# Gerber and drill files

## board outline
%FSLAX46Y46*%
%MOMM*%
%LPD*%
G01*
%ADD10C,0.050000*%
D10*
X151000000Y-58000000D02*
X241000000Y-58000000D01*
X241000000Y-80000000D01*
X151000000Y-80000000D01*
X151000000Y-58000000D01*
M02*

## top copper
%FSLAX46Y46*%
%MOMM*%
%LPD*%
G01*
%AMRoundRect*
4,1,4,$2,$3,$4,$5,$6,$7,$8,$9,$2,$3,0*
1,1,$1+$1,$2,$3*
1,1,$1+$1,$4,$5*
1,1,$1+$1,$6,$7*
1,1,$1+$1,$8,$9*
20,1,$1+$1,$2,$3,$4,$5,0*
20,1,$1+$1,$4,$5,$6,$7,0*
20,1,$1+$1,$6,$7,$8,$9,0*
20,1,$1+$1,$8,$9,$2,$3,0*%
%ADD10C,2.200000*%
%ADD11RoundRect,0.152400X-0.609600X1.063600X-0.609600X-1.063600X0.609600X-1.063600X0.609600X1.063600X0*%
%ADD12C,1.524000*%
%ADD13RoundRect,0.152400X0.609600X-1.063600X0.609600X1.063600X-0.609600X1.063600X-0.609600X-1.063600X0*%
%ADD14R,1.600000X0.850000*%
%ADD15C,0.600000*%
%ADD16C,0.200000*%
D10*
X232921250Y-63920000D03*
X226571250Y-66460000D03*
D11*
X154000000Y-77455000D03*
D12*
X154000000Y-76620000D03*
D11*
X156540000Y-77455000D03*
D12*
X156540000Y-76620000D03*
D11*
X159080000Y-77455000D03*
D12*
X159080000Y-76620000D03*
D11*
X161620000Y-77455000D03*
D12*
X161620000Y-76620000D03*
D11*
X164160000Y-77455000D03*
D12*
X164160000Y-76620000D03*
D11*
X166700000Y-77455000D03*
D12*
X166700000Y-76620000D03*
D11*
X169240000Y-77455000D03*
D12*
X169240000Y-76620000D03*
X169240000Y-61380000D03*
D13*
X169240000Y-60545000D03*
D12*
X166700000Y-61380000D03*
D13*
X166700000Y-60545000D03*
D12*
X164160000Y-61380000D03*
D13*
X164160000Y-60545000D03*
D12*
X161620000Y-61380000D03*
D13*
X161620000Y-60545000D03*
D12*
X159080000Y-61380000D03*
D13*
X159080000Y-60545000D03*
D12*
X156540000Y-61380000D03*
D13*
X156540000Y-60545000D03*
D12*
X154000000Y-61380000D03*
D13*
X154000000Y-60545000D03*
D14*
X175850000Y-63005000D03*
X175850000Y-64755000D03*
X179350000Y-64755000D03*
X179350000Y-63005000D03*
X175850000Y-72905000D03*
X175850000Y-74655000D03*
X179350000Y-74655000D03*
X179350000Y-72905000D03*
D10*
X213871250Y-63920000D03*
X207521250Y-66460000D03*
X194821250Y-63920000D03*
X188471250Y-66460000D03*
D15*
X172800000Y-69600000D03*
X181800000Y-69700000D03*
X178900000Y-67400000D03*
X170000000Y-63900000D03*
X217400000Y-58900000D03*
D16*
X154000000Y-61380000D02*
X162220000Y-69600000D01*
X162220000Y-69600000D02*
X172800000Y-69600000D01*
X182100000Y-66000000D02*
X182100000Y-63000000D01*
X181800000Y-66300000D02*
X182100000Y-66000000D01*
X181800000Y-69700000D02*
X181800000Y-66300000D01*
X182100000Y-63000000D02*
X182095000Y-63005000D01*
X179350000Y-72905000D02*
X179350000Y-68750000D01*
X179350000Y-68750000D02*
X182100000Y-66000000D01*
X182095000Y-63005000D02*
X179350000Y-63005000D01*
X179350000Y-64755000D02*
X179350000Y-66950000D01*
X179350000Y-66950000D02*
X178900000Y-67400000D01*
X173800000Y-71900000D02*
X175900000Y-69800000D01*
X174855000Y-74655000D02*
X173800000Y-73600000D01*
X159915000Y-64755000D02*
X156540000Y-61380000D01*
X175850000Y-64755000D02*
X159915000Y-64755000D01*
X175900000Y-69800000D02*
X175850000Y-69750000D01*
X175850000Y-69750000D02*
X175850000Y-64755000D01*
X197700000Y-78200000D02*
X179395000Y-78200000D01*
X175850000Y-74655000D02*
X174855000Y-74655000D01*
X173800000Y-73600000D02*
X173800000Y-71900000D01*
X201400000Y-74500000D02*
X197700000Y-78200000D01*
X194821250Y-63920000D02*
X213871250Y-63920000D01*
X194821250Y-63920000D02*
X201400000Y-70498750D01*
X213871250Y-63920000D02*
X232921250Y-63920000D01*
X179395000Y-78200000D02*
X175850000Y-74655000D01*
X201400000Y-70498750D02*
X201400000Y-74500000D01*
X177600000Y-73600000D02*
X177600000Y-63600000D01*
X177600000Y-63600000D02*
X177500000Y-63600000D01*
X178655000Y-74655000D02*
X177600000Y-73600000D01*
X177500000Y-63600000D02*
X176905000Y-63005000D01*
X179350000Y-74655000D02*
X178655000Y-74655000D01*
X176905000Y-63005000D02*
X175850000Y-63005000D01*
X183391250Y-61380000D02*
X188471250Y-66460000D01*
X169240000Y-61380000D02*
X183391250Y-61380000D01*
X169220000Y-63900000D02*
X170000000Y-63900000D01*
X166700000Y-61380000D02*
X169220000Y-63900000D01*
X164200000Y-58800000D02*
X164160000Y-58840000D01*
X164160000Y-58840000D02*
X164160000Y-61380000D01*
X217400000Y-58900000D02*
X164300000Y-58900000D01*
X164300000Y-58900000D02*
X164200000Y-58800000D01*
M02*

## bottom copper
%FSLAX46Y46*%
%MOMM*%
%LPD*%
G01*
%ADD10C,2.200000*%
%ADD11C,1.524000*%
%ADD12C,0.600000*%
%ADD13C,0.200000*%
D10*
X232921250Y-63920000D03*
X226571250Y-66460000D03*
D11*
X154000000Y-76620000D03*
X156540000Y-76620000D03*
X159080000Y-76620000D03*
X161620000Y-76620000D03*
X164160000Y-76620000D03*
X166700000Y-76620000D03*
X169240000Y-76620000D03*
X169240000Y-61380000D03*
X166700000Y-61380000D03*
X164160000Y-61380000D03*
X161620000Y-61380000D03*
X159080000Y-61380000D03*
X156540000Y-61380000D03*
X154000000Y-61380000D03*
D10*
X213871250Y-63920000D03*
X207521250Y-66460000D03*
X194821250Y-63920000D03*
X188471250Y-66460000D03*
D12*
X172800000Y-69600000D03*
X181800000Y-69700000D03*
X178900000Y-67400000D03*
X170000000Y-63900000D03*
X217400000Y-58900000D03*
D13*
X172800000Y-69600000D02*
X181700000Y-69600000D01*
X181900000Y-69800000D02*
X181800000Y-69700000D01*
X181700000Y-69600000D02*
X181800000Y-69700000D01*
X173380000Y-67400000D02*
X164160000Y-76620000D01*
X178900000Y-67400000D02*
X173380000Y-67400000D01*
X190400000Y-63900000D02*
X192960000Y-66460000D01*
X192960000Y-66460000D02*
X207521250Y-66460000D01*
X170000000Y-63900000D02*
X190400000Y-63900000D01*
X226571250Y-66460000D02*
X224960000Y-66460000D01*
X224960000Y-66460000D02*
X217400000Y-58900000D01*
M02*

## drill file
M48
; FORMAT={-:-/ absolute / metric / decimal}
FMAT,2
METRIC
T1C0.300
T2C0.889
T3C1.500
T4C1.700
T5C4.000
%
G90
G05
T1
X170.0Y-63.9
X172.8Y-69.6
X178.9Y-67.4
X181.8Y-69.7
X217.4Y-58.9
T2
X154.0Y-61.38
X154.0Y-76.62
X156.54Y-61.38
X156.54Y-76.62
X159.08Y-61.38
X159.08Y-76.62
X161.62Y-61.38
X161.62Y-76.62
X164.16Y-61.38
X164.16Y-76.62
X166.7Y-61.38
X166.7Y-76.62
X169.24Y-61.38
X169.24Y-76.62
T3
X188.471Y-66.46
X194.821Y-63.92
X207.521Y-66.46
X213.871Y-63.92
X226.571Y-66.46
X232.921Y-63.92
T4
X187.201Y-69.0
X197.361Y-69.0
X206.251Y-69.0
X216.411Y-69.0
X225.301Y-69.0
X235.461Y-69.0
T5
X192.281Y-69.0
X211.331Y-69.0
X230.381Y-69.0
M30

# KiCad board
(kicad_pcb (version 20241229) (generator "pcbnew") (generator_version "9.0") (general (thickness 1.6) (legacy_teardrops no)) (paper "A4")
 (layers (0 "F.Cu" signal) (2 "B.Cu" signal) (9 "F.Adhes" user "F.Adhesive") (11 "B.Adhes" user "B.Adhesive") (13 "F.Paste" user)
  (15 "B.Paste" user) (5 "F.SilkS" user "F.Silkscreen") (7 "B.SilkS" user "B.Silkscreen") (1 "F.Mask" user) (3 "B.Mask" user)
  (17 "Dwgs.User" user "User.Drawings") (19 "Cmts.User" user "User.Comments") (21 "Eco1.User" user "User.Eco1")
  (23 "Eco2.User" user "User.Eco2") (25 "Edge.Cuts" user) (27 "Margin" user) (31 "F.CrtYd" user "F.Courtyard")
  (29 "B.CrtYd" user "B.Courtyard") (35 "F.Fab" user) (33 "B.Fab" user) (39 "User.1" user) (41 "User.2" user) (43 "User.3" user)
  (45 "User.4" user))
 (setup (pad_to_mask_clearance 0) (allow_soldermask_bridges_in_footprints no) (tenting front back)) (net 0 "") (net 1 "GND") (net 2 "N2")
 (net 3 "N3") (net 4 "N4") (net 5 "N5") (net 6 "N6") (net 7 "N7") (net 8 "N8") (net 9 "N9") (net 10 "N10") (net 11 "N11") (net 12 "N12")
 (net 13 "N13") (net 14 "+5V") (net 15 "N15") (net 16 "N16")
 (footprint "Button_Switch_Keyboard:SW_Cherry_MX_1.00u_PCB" (layer "F.Cu") (at 232.92125 63.92)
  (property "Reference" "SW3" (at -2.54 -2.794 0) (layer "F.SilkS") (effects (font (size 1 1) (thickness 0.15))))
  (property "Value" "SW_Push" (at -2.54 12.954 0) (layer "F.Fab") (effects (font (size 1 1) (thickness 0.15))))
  (pad "" np_thru_hole circle (at -7.62 5.08) (size 1.7 1.7) (drill 1.7) (layers "*.Cu" "*.Mask"))
  (pad "" np_thru_hole circle (at -2.54 5.08) (size 4 4) (drill 4) (layers "*.Cu" "*.Mask"))
  (pad "" np_thru_hole circle (at 2.54 5.08) (size 1.7 1.7) (drill 1.7) (layers "*.Cu" "*.Mask"))
  (pad "1" thru_hole circle (at 0 0) (size 2.2 2.2) (drill 1.5) (layers "*.Cu" "*.Mask") (remove_unused_layers no) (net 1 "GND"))
  (pad "2" thru_hole circle (at -6.35 2.54) (size 2.2 2.2) (drill 1.5) (layers "*.Cu" "*.Mask") (remove_unused_layers no) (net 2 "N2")))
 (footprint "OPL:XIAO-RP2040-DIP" (layer "F.Cu") (at 161.62 69 90)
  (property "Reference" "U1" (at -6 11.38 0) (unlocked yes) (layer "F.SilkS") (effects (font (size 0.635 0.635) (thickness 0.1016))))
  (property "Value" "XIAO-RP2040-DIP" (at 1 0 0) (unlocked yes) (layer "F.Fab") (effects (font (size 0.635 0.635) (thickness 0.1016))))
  (pad "1" smd roundrect (at -8.455 -7.62 270) (size 2.432 1.524) (layers "F.Cu" "F.Mask") (roundrect_rratio 0.1) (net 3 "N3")
   (thermal_bridge_angle 45))
  (pad "1" thru_hole circle (at -7.62 -7.62 270) (size 1.524 1.524) (drill 0.889) (layers "*.Cu" "*.Mask") (remove_unused_layers no)
   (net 3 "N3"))
  (pad "2" smd roundrect (at -8.455 -5.08 270) (size 2.432 1.524) (layers "F.Cu" "F.Mask") (roundrect_rratio 0.1) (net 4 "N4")
   (thermal_bridge_angle 45))
  (pad "2" thru_hole circle (at -7.62 -5.08 270) (size 1.524 1.524) (drill 0.889) (layers "*.Cu" "*.Mask") (remove_unused_layers no)
   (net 4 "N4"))
  (pad "3" smd roundrect (at -8.455 -2.54 270) (size 2.432 1.524) (layers "F.Cu" "F.Mask") (roundrect_rratio 0.1) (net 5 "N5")
   (thermal_bridge_angle 45))
  (pad "3" thru_hole circle (at -7.62 -2.54 270) (size 1.524 1.524) (drill 0.889) (layers "*.Cu" "*.Mask") (remove_unused_layers no)
   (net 5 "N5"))
  (pad "4" smd roundrect (at -8.455 0 270) (size 2.432 1.524) (layers "F.Cu" "F.Mask") (roundrect_rratio 0.1) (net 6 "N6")
   (thermal_bridge_angle 45))
  (pad "4" thru_hole circle (at -7.62 0 270) (size 1.524 1.524) (drill 0.889) (layers "*.Cu" "*.Mask") (remove_unused_layers no)
   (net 6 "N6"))
  (pad "5" smd roundrect (at -8.455 2.54 270) (size 2.432 1.524) (layers "F.Cu" "F.Mask") (roundrect_rratio 0.1) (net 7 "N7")
   (thermal_bridge_angle 45))
  (pad "5" thru_hole circle (at -7.62 2.54 270) (size 1.524 1.524) (drill 0.889) (layers "*.Cu" "*.Mask") (remove_unused_layers no)
   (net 7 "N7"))
  (pad "6" smd roundrect (at -8.455 5.08 270) (size 2.432 1.524) (layers "F.Cu" "F.Mask") (roundrect_rratio 0.1) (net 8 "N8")
   (thermal_bridge_angle 45))
  (pad "6" thru_hole circle (at -7.62 5.08 270) (size 1.524 1.524) (drill 0.889) (layers "*.Cu" "*.Mask") (remove_unused_layers no)
   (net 8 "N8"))
  (pad "7" smd roundrect (at -8.455 7.62 270) (size 2.432 1.524) (layers "F.Cu" "F.Mask") (roundrect_rratio 0.1) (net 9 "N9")
   (thermal_bridge_angle 45))
  (pad "7" thru_hole circle (at -7.62 7.62 270) (size 1.524 1.524) (drill 0.889) (layers "*.Cu" "*.Mask") (remove_unused_layers no)
   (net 9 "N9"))
  (pad "8" thru_hole circle (at 7.62 7.62 90) (size 1.524 1.524) (drill 0.889) (layers "*.Cu" "*.Mask") (remove_unused_layers no)
   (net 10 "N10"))
  (pad "8" smd roundrect (at 8.455 7.62 90) (size 2.432 1.524) (layers "F.Cu" "F.Mask") (roundrect_rratio 0.1) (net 10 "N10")
   (thermal_bridge_angle 45))
  (pad "9" thru_hole circle (at 7.62 5.08 90) (size 1.524 1.524) (drill 0.889) (layers "*.Cu" "*.Mask") (remove_unused_layers no)
   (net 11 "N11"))
  (pad "9" smd roundrect (at 8.455 5.08 90) (size 2.432 1.524) (layers "F.Cu" "F.Mask") (roundrect_rratio 0.1) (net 11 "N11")
   (thermal_bridge_angle 45))
  (pad "10" thru_hole circle (at 7.62 2.54 90) (size 1.524 1.524) (drill 0.889) (layers "*.Cu" "*.Mask") (remove_unused_layers no)
   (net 2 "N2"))
  (pad "10" smd roundrect (at 8.455 2.54 90) (size 2.432 1.524) (layers "F.Cu" "F.Mask") (roundrect_rratio 0.1) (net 2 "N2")
   (thermal_bridge_angle 45))
  (pad "11" thru_hole circle (at 7.62 0 90) (size 1.524 1.524) (drill 0.889) (layers "*.Cu" "*.Mask") (remove_unused_layers no)
   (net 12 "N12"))
  (pad "11" smd roundrect (at 8.455 0 90) (size 2.432 1.524) (layers "F.Cu" "F.Mask") (roundrect_rratio 0.1) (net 12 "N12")
   (thermal_bridge_angle 45))
  (pad "12" thru_hole circle (at 7.62 -2.54 90) (size 1.524 1.524) (drill 0.889) (layers "*.Cu" "*.Mask") (remove_unused_layers no)
   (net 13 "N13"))
  (pad "12" smd roundrect (at 8.455 -2.54 90) (size 2.432 1.524) (layers "F.Cu" "F.Mask") (roundrect_rratio 0.1) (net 13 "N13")
   (thermal_bridge_angle 45))
  (pad "13" thru_hole circle (at 7.62 -5.08 90) (size 1.524 1.524) (drill 0.889) (layers "*.Cu" "*.Mask") (remove_unused_layers no)
   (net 1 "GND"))
  (pad "13" smd roundrect (at 8.455 -5.08 90) (size 2.432 1.524) (layers "F.Cu" "F.Mask") (roundrect_rratio 0.1) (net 1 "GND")
   (thermal_bridge_angle 45))
  (pad "14" thru_hole circle (at 7.62 -7.62 90) (size 1.524 1.524) (drill 0.889) (layers "*.Cu" "*.Mask") (remove_unused_layers no)
   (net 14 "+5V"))
  (pad "14" smd roundrect (at 8.455 -7.62 90) (size 2.432 1.524) (layers "F.Cu" "F.Mask") (roundrect_rratio 0.1) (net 14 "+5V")
   (thermal_bridge_angle 45)))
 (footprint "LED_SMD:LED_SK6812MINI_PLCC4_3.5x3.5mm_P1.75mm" (layer "F.Cu") (at 177.6 63.88)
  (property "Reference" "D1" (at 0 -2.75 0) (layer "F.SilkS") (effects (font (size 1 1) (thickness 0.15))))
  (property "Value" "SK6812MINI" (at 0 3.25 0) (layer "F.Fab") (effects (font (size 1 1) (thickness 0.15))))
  (pad "1" smd rect (at -1.75 -0.875) (size 1.6 0.85) (layers "F.Cu" "F.Mask" "F.Paste") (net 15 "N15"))
  (pad "2" smd rect (at -1.75 0.875) (size 1.6 0.85) (layers "F.Cu" "F.Mask" "F.Paste") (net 1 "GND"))
  (pad "3" smd rect (at 1.75 0.875) (size 1.6 0.85) (layers "F.Cu" "F.Mask" "F.Paste") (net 7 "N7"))
  (pad "4" smd rect (at 1.75 -0.875) (size 1.6 0.85) (layers "F.Cu" "F.Mask" "F.Paste") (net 14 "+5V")))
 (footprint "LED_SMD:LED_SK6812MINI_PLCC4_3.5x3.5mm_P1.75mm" (layer "F.Cu") (at 177.6 73.78)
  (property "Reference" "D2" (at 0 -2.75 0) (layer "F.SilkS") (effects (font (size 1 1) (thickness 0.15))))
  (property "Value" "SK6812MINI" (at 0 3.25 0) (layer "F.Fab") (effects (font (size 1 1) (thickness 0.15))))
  (pad "1" smd rect (at -1.75 -0.875) (size 1.6 0.85) (layers "F.Cu" "F.Mask" "F.Paste") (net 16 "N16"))
  (pad "2" smd rect (at -1.75 0.875) (size 1.6 0.85) (layers "F.Cu" "F.Mask" "F.Paste") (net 1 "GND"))
  (pad "3" smd rect (at 1.75 0.875) (size 1.6 0.85) (layers "F.Cu" "F.Mask" "F.Paste") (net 15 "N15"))
  (pad "4" smd rect (at 1.75 -0.875) (size 1.6 0.85) (layers "F.Cu" "F.Mask" "F.Paste") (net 14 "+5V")))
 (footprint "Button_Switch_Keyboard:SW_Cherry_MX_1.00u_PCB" (layer "F.Cu") (at 213.87125 63.92)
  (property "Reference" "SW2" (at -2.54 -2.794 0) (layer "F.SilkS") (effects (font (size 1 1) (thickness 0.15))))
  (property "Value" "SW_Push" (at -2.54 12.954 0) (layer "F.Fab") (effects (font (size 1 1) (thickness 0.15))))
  (pad "" np_thru_hole circle (at -7.62 5.08) (size 1.7 1.7) (drill 1.7) (layers "*.Cu" "*.Mask"))
  (pad "" np_thru_hole circle (at -2.54 5.08) (size 4 4) (drill 4) (layers "*.Cu" "*.Mask"))
  (pad "" np_thru_hole circle (at 2.54 5.08) (size 1.7 1.7) (drill 1.7) (layers "*.Cu" "*.Mask"))
  (pad "1" thru_hole circle (at 0 0) (size 2.2 2.2) (drill 1.5) (layers "*.Cu" "*.Mask") (remove_unused_layers no) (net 1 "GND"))
  (pad "2" thru_hole circle (at -6.35 2.54) (size 2.2 2.2) (drill 1.5) (layers "*.Cu" "*.Mask") (remove_unused_layers no) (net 11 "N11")))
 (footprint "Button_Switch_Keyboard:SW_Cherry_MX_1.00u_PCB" (layer "F.Cu") (at 194.82125 63.92)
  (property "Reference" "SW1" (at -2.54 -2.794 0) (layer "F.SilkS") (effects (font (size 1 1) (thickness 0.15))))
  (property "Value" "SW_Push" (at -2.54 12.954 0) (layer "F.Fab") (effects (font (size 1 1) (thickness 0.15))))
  (pad "" np_thru_hole circle (at -7.62 5.08) (size 1.7 1.7) (drill 1.7) (layers "*.Cu" "*.Mask"))
  (pad "" np_thru_hole circle (at -2.54 5.08) (size 4 4) (drill 4) (layers "*.Cu" "*.Mask"))
  (pad "" np_thru_hole circle (at 2.54 5.08) (size 1.7 1.7) (drill 1.7) (layers "*.Cu" "*.Mask"))
  (pad "1" thru_hole circle (at 0 0) (size 2.2 2.2) (drill 1.5) (layers "*.Cu" "*.Mask") (remove_unused_layers no) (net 1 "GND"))
  (pad "2" thru_hole circle (at -6.35 2.54) (size 2.2 2.2) (drill 1.5) (layers "*.Cu" "*.Mask") (remove_unused_layers no) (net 10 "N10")))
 (gr_rect (start 151 58) (end 241 80) (stroke (width 0.05) (type default)) (fill no) (layer "Edge.Cuts"))
 (segment (start 154 61.38) (end 162.22 69.6) (width 0.2) (layer "F.Cu") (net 14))
 (segment (start 162.22 69.6) (end 172.8 69.6) (width 0.2) (layer "F.Cu") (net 14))
 (segment (start 182.1 66) (end 182.1 63) (width 0.2) (layer "F.Cu") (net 14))
 (segment (start 181.8 66.3) (end 182.1 66) (width 0.2) (layer "F.Cu") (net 14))
 (segment (start 181.8 69.7) (end 181.8 66.3) (width 0.2) (layer "F.Cu") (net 14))
 (segment (start 182.1 63) (end 182.095 63.005) (width 0.2) (layer "F.Cu") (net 14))
 (segment (start 179.35 72.905) (end 179.35 68.75) (width 0.2) (layer "F.Cu") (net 14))
 (segment (start 179.35 68.75) (end 182.1 66) (width 0.2) (layer "F.Cu") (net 14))
 (segment (start 182.095 63.005) (end 179.35 63.005) (width 0.2) (layer "F.Cu") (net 14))
 (via (at 172.8 69.6) (size 0.6) (drill 0.3) (layers "F.Cu" "B.Cu") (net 14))
 (via (at 181.8 69.7) (size 0.6) (drill 0.3) (layers "F.Cu" "B.Cu") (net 14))
 (segment (start 172.8 69.6) (end 181.7 69.6) (width 0.2) (layer "B.Cu") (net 14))
 (segment (start 181.9 69.8) (end 181.8 69.7) (width 0.2) (layer "B.Cu") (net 14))
 (segment (start 181.7 69.6) (end 181.8 69.7) (width 0.2) (layer "B.Cu") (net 14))
 (segment (start 179.35 64.755) (end 179.35 66.95) (width 0.2) (layer "F.Cu") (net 7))
 (segment (start 179.35 66.95) (end 178.9 67.4) (width 0.2) (layer "F.Cu") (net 7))
 (via (at 178.9 67.4) (size 0.6) (drill 0.3) (layers "F.Cu" "B.Cu") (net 7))
 (segment (start 173.38 67.4) (end 164.16 76.62) (width 0.2) (layer "B.Cu") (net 7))
 (segment (start 178.9 67.4) (end 173.38 67.4) (width 0.2) (layer "B.Cu") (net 7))
 (segment (start 173.8 71.9) (end 175.9 69.8) (width 0.2) (layer "F.Cu") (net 1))
 (segment (start 174.855 74.655) (end 173.8 73.6) (width 0.2) (layer "F.Cu") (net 1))
 (segment (start 159.915 64.755) (end 156.54 61.38) (width 0.2) (layer "F.Cu") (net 1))
 (segment (start 175.85 64.755) (end 159.915 64.755) (width 0.2) (layer "F.Cu") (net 1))
 (segment (start 175.9 69.8) (end 175.85 69.75) (width 0.2) (layer "F.Cu") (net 1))
 (segment (start 175.85 69.75) (end 175.85 64.755) (width 0.2) (layer "F.Cu") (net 1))
 (segment (start 197.7 78.2) (end 179.395 78.2) (width 0.2) (layer "F.Cu") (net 1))
 (segment (start 175.85 74.655) (end 174.855 74.655) (width 0.2) (layer "F.Cu") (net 1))
 (segment (start 173.8 73.6) (end 173.8 71.9) (width 0.2) (layer "F.Cu") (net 1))
 (segment (start 201.4 74.5) (end 197.7 78.2) (width 0.2) (layer "F.Cu") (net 1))
 (segment (start 194.82125 63.92) (end 213.87125 63.92) (width 0.2) (layer "F.Cu") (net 1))
 (segment (start 194.82125 63.92) (end 201.4 70.49875) (width 0.2) (layer "F.Cu") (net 1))
 (segment (start 213.87125 63.92) (end 232.92125 63.92) (width 0.2) (layer "F.Cu") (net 1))
 (segment (start 179.395 78.2) (end 175.85 74.655) (width 0.2) (layer "F.Cu") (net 1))
 (segment (start 201.4 70.49875) (end 201.4 74.5) (width 0.2) (layer "F.Cu") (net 1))
 (segment (start 177.6 73.6) (end 177.6 63.6) (width 0.2) (layer "F.Cu") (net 15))
 (segment (start 177.6 63.6) (end 177.5 63.6) (width 0.2) (layer "F.Cu") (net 15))
 (segment (start 178.655 74.655) (end 177.6 73.6) (width 0.2) (layer "F.Cu") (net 15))
 (segment (start 177.5 63.6) (end 176.905 63.005) (width 0.2) (layer "F.Cu") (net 15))
 (segment (start 179.35 74.655) (end 178.655 74.655) (width 0.2) (layer "F.Cu") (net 15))
 (segment (start 176.905 63.005) (end 175.85 63.005) (width 0.2) (layer "F.Cu") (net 15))
 (segment (start 183.39125 61.38) (end 188.47125 66.46) (width 0.2) (layer "F.Cu") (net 10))
 (segment (start 169.24 61.38) (end 183.39125 61.38) (width 0.2) (layer "F.Cu") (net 10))
 (segment (start 169.22 63.9) (end 170 63.9) (width 0.2) (layer "F.Cu") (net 11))
 (segment (start 166.7 61.38) (end 169.22 63.9) (width 0.2) (layer "F.Cu") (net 11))
 (via (at 170 63.9) (size 0.6) (drill 0.3) (layers "F.Cu" "B.Cu") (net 11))
 (segment (start 190.4 63.9) (end 192.96 66.46) (width 0.2) (layer "B.Cu") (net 11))
 (segment (start 192.96 66.46) (end 207.52125 66.46) (width 0.2) (layer "B.Cu") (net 11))
 (segment (start 170 63.9) (end 190.4 63.9) (width 0.2) (layer "B.Cu") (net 11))
 (segment (start 164.2 58.8) (end 164.16 58.84) (width 0.2) (layer "F.Cu") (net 2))
 (segment (start 164.16 58.84) (end 164.16 61.38) (width 0.2) (layer "F.Cu") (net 2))
 (segment (start 217.4 58.9) (end 164.3 58.9) (width 0.2) (layer "F.Cu") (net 2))
 (segment (start 164.3 58.9) (end 164.2 58.8) (width 0.2) (layer "F.Cu") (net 2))
 (via (at 217.4 58.9) (size 0.6) (drill 0.3) (layers "F.Cu" "B.Cu") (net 2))
 (segment (start 226.57125 66.46) (end 224.96 66.46) (width 0.2) (layer "B.Cu") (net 2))
 (segment (start 224.96 66.46) (end 217.4 58.9) (width 0.2) (layer "B.Cu") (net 2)))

